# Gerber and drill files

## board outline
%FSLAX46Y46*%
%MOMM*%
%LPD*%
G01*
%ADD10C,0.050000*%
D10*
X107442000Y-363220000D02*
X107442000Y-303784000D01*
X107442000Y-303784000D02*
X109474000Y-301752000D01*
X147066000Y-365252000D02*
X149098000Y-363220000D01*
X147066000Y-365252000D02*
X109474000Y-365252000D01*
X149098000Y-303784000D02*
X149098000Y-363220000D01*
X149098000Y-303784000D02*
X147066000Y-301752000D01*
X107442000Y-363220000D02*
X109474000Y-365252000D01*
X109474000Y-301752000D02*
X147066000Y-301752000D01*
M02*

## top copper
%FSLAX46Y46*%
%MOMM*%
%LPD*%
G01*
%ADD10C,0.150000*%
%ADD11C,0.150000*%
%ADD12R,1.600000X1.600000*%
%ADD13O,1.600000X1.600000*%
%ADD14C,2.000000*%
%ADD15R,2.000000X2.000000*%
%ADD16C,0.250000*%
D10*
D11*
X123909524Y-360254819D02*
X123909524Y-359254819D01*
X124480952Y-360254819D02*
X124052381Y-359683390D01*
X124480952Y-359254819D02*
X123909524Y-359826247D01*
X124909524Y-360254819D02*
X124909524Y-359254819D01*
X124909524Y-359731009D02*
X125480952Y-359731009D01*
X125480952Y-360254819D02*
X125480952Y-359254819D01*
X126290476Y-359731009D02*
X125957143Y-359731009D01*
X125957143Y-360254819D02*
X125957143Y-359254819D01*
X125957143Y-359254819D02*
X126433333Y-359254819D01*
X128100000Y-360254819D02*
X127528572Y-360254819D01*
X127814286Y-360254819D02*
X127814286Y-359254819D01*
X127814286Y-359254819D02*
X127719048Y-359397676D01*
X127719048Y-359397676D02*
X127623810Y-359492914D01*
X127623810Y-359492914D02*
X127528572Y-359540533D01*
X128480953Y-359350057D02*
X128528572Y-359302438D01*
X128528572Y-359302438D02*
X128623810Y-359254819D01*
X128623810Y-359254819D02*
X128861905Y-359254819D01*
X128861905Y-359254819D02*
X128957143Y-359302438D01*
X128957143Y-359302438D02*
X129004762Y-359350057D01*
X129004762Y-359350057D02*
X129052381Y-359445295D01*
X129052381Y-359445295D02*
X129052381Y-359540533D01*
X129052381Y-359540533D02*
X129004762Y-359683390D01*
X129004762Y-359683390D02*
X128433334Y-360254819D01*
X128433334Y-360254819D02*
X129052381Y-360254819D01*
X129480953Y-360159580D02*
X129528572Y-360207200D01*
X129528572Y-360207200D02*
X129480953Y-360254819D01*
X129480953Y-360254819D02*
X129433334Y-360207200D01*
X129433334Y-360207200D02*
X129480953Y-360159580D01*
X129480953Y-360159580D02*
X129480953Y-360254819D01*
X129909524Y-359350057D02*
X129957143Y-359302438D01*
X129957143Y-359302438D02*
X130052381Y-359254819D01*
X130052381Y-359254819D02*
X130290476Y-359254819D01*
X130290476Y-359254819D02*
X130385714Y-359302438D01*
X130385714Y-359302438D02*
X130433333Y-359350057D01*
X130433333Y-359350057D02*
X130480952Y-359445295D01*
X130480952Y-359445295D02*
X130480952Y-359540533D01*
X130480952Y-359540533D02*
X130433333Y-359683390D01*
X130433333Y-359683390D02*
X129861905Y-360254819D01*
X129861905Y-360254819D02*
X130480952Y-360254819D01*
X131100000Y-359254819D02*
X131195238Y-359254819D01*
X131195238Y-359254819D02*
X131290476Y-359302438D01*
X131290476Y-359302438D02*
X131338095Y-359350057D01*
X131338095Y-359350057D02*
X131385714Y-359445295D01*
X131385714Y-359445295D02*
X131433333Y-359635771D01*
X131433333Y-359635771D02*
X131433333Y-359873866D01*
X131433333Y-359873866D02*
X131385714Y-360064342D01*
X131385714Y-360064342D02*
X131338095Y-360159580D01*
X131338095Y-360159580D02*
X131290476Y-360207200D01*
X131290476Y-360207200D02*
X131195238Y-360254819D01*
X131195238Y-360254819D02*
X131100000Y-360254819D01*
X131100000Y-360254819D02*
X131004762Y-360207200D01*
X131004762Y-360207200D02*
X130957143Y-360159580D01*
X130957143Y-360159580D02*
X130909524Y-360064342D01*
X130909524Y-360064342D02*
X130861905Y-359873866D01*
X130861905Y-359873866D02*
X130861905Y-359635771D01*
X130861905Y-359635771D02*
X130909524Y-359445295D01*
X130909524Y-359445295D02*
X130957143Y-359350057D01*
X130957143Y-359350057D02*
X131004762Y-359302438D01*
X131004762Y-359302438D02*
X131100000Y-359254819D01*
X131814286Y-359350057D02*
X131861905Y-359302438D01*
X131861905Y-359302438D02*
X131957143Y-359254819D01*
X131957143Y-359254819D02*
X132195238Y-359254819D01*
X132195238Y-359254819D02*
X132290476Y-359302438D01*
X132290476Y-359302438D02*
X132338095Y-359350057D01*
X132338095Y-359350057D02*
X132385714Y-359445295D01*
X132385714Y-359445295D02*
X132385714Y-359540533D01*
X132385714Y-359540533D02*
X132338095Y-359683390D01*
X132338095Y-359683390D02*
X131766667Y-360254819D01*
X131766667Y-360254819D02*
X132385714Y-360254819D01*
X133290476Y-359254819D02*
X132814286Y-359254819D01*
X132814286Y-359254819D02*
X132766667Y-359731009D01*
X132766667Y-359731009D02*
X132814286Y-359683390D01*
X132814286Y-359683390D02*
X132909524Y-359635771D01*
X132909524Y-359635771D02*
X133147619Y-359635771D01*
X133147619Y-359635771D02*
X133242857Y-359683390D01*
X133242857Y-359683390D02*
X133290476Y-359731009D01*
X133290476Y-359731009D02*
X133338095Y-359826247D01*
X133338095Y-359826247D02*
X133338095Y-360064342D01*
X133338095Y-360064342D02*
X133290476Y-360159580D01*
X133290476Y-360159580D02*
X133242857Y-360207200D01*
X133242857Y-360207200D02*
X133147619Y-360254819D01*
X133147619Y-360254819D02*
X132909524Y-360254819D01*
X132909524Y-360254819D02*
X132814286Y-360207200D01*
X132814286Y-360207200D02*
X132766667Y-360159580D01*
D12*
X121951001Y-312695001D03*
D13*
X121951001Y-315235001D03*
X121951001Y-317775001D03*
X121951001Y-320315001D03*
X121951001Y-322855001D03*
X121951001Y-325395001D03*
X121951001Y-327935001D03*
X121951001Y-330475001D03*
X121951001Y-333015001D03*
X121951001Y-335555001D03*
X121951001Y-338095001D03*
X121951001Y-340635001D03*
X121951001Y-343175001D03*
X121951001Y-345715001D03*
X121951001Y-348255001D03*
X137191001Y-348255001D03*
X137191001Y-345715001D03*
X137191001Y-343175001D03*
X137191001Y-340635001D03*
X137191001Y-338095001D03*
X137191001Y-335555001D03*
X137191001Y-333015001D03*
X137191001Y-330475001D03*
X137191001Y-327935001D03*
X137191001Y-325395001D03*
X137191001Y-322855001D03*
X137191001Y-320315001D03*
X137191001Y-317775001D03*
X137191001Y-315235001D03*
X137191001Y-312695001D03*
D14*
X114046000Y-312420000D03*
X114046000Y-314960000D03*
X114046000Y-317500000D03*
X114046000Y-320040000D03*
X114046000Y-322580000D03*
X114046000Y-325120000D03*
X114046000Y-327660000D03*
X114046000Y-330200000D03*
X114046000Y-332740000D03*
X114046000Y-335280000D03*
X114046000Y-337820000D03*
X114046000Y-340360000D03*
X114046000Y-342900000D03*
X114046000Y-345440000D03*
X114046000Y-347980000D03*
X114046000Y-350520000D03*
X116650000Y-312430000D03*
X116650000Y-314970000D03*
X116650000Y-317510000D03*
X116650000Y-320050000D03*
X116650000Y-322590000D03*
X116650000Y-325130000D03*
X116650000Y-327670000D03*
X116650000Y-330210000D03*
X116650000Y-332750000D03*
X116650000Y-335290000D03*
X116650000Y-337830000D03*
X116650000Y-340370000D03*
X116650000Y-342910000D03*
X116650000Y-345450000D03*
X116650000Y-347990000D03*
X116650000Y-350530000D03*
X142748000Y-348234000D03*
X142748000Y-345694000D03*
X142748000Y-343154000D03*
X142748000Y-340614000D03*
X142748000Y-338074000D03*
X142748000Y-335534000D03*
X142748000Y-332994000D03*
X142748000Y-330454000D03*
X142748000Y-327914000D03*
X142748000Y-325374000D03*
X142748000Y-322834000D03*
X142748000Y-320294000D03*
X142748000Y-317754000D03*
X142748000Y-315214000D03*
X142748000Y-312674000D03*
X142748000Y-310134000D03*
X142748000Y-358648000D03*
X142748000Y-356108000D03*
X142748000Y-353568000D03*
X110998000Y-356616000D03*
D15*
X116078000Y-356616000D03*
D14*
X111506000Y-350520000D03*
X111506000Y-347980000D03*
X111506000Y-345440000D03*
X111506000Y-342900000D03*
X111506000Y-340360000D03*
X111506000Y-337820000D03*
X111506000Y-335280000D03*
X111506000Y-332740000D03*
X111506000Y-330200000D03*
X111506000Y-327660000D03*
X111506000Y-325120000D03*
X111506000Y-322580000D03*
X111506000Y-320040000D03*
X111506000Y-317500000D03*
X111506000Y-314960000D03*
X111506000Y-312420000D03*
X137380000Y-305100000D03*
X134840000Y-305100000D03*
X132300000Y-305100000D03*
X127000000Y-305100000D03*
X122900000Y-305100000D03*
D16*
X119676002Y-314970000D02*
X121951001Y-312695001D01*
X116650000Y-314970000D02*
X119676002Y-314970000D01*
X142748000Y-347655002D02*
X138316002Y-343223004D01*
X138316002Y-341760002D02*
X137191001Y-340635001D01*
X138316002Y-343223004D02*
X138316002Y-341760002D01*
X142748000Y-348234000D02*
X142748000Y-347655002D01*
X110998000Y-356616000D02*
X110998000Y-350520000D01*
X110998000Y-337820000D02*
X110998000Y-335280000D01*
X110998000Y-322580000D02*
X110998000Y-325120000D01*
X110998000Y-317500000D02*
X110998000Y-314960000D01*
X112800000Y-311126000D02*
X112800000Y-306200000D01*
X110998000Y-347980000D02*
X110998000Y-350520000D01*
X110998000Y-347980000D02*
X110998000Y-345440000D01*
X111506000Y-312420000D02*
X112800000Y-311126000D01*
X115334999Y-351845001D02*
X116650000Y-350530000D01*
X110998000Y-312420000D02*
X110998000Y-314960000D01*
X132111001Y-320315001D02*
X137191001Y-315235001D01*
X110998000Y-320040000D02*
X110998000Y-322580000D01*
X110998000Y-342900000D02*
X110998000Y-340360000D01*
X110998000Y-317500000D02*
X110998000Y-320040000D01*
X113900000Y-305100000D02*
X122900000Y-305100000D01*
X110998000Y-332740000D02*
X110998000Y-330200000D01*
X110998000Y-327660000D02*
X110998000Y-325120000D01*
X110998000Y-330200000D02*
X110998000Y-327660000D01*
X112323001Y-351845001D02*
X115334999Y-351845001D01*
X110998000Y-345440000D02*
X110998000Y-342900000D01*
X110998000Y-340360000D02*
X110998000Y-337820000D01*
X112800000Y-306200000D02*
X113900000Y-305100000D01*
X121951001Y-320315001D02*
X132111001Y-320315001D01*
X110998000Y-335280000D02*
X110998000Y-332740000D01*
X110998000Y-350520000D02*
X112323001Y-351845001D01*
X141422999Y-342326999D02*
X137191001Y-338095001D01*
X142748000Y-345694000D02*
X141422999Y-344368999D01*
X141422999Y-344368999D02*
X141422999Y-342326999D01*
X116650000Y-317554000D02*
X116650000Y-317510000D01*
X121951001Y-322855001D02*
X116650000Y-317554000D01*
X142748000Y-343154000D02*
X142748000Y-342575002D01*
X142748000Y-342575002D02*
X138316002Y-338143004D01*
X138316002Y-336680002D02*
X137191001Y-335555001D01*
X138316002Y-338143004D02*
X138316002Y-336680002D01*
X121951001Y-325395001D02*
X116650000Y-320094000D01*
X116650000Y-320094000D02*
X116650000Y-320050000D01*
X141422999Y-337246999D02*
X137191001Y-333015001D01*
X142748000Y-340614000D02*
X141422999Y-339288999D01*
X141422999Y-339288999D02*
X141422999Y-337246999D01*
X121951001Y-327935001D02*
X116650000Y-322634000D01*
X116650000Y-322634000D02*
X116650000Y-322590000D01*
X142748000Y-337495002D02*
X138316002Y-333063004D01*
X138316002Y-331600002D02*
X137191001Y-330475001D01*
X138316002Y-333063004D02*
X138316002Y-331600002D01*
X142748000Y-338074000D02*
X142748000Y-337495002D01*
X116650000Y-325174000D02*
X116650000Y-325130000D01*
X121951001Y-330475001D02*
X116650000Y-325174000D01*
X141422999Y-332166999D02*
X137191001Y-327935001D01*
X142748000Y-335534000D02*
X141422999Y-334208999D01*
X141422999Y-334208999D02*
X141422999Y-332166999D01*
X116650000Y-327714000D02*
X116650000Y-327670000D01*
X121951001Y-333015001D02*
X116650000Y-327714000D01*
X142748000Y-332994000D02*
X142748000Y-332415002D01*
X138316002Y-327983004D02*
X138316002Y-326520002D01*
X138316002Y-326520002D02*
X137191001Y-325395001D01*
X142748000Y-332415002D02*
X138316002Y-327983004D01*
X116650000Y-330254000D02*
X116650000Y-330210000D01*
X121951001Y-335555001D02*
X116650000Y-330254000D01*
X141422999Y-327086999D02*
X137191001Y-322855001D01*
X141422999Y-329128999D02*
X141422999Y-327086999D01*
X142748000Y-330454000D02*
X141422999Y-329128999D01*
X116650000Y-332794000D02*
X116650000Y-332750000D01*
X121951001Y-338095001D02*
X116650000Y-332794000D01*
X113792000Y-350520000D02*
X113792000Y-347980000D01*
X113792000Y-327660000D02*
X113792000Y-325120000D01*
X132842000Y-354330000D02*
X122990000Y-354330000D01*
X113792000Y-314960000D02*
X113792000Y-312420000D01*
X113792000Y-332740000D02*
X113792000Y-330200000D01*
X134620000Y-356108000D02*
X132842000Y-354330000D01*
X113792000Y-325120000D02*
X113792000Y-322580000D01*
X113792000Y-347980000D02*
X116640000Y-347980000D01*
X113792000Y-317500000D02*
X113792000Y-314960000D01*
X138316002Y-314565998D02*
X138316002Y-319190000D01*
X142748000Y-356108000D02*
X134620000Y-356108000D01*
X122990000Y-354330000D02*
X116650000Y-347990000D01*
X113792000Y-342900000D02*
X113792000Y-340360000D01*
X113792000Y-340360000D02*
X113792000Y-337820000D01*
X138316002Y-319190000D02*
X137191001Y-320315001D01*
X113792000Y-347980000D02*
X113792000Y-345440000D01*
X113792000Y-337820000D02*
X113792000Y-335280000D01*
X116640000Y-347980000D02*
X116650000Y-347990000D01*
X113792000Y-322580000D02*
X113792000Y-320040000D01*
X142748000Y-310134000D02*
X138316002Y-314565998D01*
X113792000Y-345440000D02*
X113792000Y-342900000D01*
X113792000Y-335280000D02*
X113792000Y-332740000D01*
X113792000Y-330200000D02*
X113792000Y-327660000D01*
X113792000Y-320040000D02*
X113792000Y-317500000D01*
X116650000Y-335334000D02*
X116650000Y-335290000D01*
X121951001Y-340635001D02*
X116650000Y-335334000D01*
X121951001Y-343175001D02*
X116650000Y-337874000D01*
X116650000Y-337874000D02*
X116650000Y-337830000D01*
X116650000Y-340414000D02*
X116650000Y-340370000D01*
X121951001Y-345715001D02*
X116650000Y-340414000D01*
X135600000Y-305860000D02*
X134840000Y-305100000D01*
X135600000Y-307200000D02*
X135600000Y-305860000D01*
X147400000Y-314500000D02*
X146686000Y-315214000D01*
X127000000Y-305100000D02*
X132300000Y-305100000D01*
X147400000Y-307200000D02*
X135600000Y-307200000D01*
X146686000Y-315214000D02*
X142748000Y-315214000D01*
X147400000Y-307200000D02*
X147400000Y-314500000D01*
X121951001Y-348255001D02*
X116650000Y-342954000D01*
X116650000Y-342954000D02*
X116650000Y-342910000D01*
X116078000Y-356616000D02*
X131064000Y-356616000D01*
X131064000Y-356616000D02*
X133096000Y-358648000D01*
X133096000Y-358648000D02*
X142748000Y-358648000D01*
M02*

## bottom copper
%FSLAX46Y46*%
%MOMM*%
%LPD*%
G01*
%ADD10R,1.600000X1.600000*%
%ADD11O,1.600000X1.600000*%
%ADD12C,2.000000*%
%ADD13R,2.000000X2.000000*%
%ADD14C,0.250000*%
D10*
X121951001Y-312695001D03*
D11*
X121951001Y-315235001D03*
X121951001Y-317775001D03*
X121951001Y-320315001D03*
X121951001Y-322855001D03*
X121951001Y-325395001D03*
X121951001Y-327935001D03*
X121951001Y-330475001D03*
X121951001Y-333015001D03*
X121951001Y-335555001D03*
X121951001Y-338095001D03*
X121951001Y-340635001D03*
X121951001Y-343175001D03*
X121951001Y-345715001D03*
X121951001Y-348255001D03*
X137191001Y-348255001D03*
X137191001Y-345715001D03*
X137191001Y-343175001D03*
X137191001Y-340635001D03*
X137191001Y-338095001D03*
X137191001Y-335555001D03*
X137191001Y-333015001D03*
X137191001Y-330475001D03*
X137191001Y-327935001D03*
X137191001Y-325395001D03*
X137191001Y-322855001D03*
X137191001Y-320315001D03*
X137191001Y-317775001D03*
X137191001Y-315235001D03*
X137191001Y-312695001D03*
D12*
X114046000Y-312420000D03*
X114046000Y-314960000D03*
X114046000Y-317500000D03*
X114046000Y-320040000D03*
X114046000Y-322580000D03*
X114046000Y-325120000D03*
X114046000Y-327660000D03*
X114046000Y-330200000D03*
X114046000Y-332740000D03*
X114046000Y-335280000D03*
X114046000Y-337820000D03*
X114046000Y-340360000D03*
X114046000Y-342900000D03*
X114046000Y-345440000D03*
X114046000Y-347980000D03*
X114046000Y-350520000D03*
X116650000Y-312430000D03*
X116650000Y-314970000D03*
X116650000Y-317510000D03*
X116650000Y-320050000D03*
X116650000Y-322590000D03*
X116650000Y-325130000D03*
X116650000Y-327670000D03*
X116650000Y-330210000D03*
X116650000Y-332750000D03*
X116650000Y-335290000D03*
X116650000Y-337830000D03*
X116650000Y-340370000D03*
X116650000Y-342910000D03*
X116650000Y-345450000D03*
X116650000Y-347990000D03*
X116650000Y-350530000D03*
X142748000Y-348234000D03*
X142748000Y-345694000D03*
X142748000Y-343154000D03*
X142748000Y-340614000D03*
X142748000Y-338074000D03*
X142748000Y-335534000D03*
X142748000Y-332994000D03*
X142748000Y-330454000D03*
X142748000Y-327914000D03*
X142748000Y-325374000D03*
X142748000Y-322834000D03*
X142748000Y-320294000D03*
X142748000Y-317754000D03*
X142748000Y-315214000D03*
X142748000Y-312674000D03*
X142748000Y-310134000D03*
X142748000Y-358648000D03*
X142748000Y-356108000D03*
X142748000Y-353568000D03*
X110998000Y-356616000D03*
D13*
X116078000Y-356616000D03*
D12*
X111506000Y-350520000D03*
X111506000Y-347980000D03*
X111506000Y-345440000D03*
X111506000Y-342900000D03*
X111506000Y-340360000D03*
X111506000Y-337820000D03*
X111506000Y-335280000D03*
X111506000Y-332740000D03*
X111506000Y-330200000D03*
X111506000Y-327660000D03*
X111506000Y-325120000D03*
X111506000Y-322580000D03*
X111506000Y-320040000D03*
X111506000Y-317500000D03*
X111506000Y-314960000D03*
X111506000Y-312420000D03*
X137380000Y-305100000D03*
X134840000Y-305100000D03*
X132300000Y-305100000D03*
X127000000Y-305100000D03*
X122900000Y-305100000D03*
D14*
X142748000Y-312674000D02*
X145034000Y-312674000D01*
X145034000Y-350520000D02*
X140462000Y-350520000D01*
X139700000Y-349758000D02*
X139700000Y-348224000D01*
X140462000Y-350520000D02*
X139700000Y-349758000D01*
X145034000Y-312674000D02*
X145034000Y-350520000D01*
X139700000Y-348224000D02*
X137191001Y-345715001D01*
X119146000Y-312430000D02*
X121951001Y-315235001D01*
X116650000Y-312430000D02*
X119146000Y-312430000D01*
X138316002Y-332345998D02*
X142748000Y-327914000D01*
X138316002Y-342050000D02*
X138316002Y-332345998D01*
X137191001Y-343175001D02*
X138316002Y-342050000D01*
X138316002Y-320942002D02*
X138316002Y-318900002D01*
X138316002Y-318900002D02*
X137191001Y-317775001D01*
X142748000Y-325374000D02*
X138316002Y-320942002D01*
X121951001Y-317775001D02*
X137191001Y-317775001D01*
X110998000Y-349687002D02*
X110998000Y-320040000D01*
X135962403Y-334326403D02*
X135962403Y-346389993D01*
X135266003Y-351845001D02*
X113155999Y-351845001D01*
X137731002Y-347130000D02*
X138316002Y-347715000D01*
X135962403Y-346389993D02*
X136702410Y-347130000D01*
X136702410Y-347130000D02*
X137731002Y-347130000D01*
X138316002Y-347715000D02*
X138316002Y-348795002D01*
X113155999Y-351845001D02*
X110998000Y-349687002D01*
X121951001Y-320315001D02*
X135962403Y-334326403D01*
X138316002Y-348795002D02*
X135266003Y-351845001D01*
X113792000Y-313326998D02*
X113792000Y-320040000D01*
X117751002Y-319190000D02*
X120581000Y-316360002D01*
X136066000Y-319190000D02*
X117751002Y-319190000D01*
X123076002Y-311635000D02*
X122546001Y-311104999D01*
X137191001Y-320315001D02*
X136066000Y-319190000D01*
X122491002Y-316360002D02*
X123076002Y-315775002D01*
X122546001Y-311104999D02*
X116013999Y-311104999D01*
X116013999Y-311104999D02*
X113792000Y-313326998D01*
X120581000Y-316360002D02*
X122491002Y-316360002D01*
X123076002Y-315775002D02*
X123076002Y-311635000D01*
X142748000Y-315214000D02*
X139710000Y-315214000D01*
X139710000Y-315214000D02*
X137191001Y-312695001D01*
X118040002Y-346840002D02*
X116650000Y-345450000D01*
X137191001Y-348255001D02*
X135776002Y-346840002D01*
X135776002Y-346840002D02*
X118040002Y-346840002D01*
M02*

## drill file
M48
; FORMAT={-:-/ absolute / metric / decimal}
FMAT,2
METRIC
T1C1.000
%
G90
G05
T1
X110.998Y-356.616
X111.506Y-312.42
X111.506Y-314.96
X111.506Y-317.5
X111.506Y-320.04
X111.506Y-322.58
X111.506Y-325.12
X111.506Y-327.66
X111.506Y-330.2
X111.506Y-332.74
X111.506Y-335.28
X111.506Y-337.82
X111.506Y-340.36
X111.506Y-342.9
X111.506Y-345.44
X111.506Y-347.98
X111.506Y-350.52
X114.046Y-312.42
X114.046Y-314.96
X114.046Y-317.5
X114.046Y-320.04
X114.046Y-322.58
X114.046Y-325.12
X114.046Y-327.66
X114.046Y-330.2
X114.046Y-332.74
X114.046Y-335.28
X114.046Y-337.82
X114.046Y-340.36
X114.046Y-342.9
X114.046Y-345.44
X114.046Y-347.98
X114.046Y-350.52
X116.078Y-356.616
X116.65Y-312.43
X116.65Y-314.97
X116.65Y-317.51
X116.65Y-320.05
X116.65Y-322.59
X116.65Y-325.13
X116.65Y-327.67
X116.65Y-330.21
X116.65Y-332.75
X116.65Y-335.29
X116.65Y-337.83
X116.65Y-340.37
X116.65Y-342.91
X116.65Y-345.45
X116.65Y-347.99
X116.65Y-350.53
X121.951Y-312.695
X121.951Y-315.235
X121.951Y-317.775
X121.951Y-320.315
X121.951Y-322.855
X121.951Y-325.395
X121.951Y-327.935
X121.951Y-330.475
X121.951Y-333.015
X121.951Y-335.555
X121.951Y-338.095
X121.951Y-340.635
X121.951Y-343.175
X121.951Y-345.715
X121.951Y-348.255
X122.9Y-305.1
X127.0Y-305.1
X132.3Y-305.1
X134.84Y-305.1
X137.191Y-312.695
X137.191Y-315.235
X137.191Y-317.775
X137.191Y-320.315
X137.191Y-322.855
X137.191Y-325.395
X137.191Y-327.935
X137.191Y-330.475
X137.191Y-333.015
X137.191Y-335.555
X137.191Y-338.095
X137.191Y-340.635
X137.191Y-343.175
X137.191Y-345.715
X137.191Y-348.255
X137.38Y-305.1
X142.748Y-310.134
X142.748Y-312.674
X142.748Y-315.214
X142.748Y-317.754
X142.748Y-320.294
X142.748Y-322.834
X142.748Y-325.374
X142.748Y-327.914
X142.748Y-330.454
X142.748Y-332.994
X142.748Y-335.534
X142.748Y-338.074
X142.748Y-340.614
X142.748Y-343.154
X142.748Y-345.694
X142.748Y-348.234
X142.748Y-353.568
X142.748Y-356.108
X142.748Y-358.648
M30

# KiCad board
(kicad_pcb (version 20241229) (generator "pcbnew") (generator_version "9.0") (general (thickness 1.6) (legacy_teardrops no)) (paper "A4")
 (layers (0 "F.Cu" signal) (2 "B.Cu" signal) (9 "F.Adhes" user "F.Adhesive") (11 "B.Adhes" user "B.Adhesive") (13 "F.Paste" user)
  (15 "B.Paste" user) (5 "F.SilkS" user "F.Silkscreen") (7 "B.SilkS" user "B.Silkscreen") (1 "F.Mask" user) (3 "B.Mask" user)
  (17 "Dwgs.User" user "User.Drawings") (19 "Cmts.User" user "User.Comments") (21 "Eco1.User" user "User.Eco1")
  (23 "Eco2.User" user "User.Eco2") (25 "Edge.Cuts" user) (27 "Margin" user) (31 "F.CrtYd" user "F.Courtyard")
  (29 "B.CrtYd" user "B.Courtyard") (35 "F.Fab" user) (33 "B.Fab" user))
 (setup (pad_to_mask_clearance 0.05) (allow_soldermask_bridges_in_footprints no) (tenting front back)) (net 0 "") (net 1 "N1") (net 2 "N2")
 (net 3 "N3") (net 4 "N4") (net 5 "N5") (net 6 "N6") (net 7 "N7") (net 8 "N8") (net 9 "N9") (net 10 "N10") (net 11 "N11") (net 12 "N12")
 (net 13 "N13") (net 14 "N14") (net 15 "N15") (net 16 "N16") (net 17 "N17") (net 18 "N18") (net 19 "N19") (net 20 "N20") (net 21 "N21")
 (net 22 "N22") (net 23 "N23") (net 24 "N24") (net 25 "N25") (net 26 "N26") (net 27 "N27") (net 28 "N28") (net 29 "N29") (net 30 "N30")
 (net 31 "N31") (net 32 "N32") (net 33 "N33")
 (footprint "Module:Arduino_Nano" (layer "F.Cu") (at 121.951001 312.695001)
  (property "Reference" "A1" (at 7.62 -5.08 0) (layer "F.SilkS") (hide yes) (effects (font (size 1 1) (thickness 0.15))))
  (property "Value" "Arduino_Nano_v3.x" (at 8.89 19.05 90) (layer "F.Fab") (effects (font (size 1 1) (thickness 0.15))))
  (pad "1" thru_hole rect (at 0 0) (size 1.6 1.6) (drill 1) (layers "*.Cu" "*.Mask") (remove_unused_layers no) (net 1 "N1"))
  (pad "2" thru_hole oval (at 0 2.54) (size 1.6 1.6) (drill 1) (layers "*.Cu" "*.Mask") (remove_unused_layers no) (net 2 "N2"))
  (pad "3" thru_hole oval (at 0 5.08) (size 1.6 1.6) (drill 1) (layers "*.Cu" "*.Mask") (remove_unused_layers no) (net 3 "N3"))
  (pad "4" thru_hole oval (at 0 7.62) (size 1.6 1.6) (drill 1) (layers "*.Cu" "*.Mask") (remove_unused_layers no) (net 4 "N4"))
  (pad "5" thru_hole oval (at 0 10.16) (size 1.6 1.6) (drill 1) (layers "*.Cu" "*.Mask") (remove_unused_layers no) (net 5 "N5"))
  (pad "6" thru_hole oval (at 0 12.7) (size 1.6 1.6) (drill 1) (layers "*.Cu" "*.Mask") (remove_unused_layers no) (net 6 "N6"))
  (pad "7" thru_hole oval (at 0 15.24) (size 1.6 1.6) (drill 1) (layers "*.Cu" "*.Mask") (remove_unused_layers no) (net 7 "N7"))
  (pad "8" thru_hole oval (at 0 17.78) (size 1.6 1.6) (drill 1) (layers "*.Cu" "*.Mask") (remove_unused_layers no) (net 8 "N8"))
  (pad "9" thru_hole oval (at 0 20.32) (size 1.6 1.6) (drill 1) (layers "*.Cu" "*.Mask") (remove_unused_layers no) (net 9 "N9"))
  (pad "10" thru_hole oval (at 0 22.86) (size 1.6 1.6) (drill 1) (layers "*.Cu" "*.Mask") (remove_unused_layers no) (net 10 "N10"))
  (pad "11" thru_hole oval (at 0 25.4) (size 1.6 1.6) (drill 1) (layers "*.Cu" "*.Mask") (remove_unused_layers no) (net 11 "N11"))
  (pad "12" thru_hole oval (at 0 27.94) (size 1.6 1.6) (drill 1) (layers "*.Cu" "*.Mask") (remove_unused_layers no) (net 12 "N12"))
  (pad "13" thru_hole oval (at 0 30.48) (size 1.6 1.6) (drill 1) (layers "*.Cu" "*.Mask") (remove_unused_layers no) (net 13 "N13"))
  (pad "14" thru_hole oval (at 0 33.02) (size 1.6 1.6) (drill 1) (layers "*.Cu" "*.Mask") (remove_unused_layers no) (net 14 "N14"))
  (pad "15" thru_hole oval (at 0 35.56) (size 1.6 1.6) (drill 1) (layers "*.Cu" "*.Mask") (remove_unused_layers no) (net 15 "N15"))
  (pad "16" thru_hole oval (at 15.24 35.56) (size 1.6 1.6) (drill 1) (layers "*.Cu" "*.Mask") (remove_unused_layers no) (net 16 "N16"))
  (pad "17" thru_hole oval (at 15.24 33.02) (size 1.6 1.6) (drill 1) (layers "*.Cu" "*.Mask") (remove_unused_layers no) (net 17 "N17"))
  (pad "18" thru_hole oval (at 15.24 30.48) (size 1.6 1.6) (drill 1) (layers "*.Cu" "*.Mask") (remove_unused_layers no) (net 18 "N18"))
  (pad "19" thru_hole oval (at 15.24 27.94) (size 1.6 1.6) (drill 1) (layers "*.Cu" "*.Mask") (remove_unused_layers no) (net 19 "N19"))
  (pad "20" thru_hole oval (at 15.24 25.4) (size 1.6 1.6) (drill 1) (layers "*.Cu" "*.Mask") (remove_unused_layers no) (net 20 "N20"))
  (pad "21" thru_hole oval (at 15.24 22.86) (size 1.6 1.6) (drill 1) (layers "*.Cu" "*.Mask") (remove_unused_layers no) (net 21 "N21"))
  (pad "22" thru_hole oval (at 15.24 20.32) (size 1.6 1.6) (drill 1) (layers "*.Cu" "*.Mask") (remove_unused_layers no) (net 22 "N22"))
  (pad "23" thru_hole oval (at 15.24 17.78) (size 1.6 1.6) (drill 1) (layers "*.Cu" "*.Mask") (remove_unused_layers no) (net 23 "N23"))
  (pad "24" thru_hole oval (at 15.24 15.24) (size 1.6 1.6) (drill 1) (layers "*.Cu" "*.Mask") (remove_unused_layers no) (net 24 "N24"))
  (pad "25" thru_hole oval (at 15.24 12.7) (size 1.6 1.6) (drill 1) (layers "*.Cu" "*.Mask") (remove_unused_layers no) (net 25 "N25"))
  (pad "26" thru_hole oval (at 15.24 10.16) (size 1.6 1.6) (drill 1) (layers "*.Cu" "*.Mask") (remove_unused_layers no) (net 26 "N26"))
  (pad "27" thru_hole oval (at 15.24 7.62) (size 1.6 1.6) (drill 1) (layers "*.Cu" "*.Mask") (remove_unused_layers no) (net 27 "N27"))
  (pad "28" thru_hole oval (at 15.24 5.08) (size 1.6 1.6) (drill 1) (layers "*.Cu" "*.Mask") (remove_unused_layers no) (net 3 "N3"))
  (pad "29" thru_hole oval (at 15.24 2.54) (size 1.6 1.6) (drill 1) (layers "*.Cu" "*.Mask") (remove_unused_layers no) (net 4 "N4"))
  (pad "30" thru_hole oval (at 15.24 0) (size 1.6 1.6) (drill 1) (layers "*.Cu" "*.Mask") (remove_unused_layers no) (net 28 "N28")))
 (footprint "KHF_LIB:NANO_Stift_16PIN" (layer "F.Cu") (at 114.046 312.42 -90)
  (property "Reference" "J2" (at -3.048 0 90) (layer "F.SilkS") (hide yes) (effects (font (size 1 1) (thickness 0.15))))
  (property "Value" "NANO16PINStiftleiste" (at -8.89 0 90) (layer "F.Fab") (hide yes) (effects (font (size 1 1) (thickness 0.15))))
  (pad "1" thru_hole circle (at 0 0 270) (size 2 2) (drill 1) (layers "*.Cu" "*.Mask") (remove_unused_layers no) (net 27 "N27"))
  (pad "2" thru_hole circle (at 2.54 0 270) (size 2 2) (drill 1) (layers "*.Cu" "*.Mask") (remove_unused_layers no) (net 27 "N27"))
  (pad "3" thru_hole circle (at 5.08 0 270) (size 2 2) (drill 1) (layers "*.Cu" "*.Mask") (remove_unused_layers no) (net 27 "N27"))
  (pad "4" thru_hole circle (at 7.62 0 270) (size 2 2) (drill 1) (layers "*.Cu" "*.Mask") (remove_unused_layers no) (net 27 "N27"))
  (pad "5" thru_hole circle (at 10.16 0 270) (size 2 2) (drill 1) (layers "*.Cu" "*.Mask") (remove_unused_layers no) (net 27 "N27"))
  (pad "6" thru_hole circle (at 12.7 0 270) (size 2 2) (drill 1) (layers "*.Cu" "*.Mask") (remove_unused_layers no) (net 27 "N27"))
  (pad "7" thru_hole circle (at 15.24 0 270) (size 2 2) (drill 1) (layers "*.Cu" "*.Mask") (remove_unused_layers no) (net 27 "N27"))
  (pad "8" thru_hole circle (at 17.78 0 270) (size 2 2) (drill 1) (layers "*.Cu" "*.Mask") (remove_unused_layers no) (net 27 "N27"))
  (pad "9" thru_hole circle (at 20.32 0 270) (size 2 2) (drill 1) (layers "*.Cu" "*.Mask") (remove_unused_layers no) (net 27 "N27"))
  (pad "10" thru_hole circle (at 22.86 0 270) (size 2 2) (drill 1) (layers "*.Cu" "*.Mask") (remove_unused_layers no) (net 27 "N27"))
  (pad "11" thru_hole circle (at 25.4 0 270) (size 2 2) (drill 1) (layers "*.Cu" "*.Mask") (remove_unused_layers no) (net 27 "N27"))
  (pad "12" thru_hole circle (at 27.94 0 270) (size 2 2) (drill 1) (layers "*.Cu" "*.Mask") (remove_unused_layers no) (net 27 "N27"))
  (pad "13" thru_hole circle (at 30.48 0 270) (size 2 2) (drill 1) (layers "*.Cu" "*.Mask") (remove_unused_layers no) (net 27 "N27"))
  (pad "14" thru_hole circle (at 33.02 0 270) (size 2 2) (drill 1) (layers "*.Cu" "*.Mask") (remove_unused_layers no) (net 27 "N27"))
  (pad "15" thru_hole circle (at 35.56 0 270) (size 2 2) (drill 1) (layers "*.Cu" "*.Mask") (remove_unused_layers no) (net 27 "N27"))
  (pad "16" thru_hole circle (at 38.1 0 270) (size 2 2) (drill 1) (layers "*.Cu" "*.Mask") (remove_unused_layers no) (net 27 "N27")))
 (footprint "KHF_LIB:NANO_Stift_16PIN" (layer "F.Cu") (at 116.65 312.43 -90)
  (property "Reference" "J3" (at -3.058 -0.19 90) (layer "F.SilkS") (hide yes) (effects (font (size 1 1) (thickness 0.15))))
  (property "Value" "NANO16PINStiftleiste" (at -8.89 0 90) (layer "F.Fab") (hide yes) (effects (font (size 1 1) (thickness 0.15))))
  (pad "1" thru_hole circle (at 0 0 270) (size 2 2) (drill 1) (layers "*.Cu" "*.Mask") (remove_unused_layers no) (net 2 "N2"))
  (pad "2" thru_hole circle (at 2.54 0 270) (size 2 2) (drill 1) (layers "*.Cu" "*.Mask") (remove_unused_layers no) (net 1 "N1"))
  (pad "3" thru_hole circle (at 5.08 0 270) (size 2 2) (drill 1) (layers "*.Cu" "*.Mask") (remove_unused_layers no) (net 5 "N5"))
  (pad "4" thru_hole circle (at 7.62 0 270) (size 2 2) (drill 1) (layers "*.Cu" "*.Mask") (remove_unused_layers no) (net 6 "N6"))
  (pad "5" thru_hole circle (at 10.16 0 270) (size 2 2) (drill 1) (layers "*.Cu" "*.Mask") (remove_unused_layers no) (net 7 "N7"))
  (pad "6" thru_hole circle (at 12.7 0 270) (size 2 2) (drill 1) (layers "*.Cu" "*.Mask") (remove_unused_layers no) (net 8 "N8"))
  (pad "7" thru_hole circle (at 15.24 0 270) (size 2 2) (drill 1) (layers "*.Cu" "*.Mask") (remove_unused_layers no) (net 9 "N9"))
  (pad "8" thru_hole circle (at 17.78 0 270) (size 2 2) (drill 1) (layers "*.Cu" "*.Mask") (remove_unused_layers no) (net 10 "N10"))
  (pad "9" thru_hole circle (at 20.32 0 270) (size 2 2) (drill 1) (layers "*.Cu" "*.Mask") (remove_unused_layers no) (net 11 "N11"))
  (pad "10" thru_hole circle (at 22.86 0 270) (size 2 2) (drill 1) (layers "*.Cu" "*.Mask") (remove_unused_layers no) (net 12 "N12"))
  (pad "11" thru_hole circle (at 25.4 0 270) (size 2 2) (drill 1) (layers "*.Cu" "*.Mask") (remove_unused_layers no) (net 13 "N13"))
  (pad "12" thru_hole circle (at 27.94 0 270) (size 2 2) (drill 1) (layers "*.Cu" "*.Mask") (remove_unused_layers no) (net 14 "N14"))
  (pad "13" thru_hole circle (at 30.48 0 270) (size 2 2) (drill 1) (layers "*.Cu" "*.Mask") (remove_unused_layers no) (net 15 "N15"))
  (pad "14" thru_hole circle (at 33.02 0 270) (size 2 2) (drill 1) (layers "*.Cu" "*.Mask") (remove_unused_layers no) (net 16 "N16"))
  (pad "15" thru_hole circle (at 35.56 0 270) (size 2 2) (drill 1) (layers "*.Cu" "*.Mask") (remove_unused_layers no) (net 27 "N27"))
  (pad "16" thru_hole circle (at 38.1 0 270) (size 2 2) (drill 1) (layers "*.Cu" "*.Mask") (remove_unused_layers no) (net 4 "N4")))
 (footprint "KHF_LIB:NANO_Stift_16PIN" (layer "F.Cu") (at 142.748 348.234 90)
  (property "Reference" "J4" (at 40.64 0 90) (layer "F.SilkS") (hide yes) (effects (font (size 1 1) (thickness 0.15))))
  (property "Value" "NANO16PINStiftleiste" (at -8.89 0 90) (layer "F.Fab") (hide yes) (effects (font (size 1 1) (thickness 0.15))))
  (pad "1" thru_hole circle (at 0 0 90) (size 2 2) (drill 1) (layers "*.Cu" "*.Mask") (remove_unused_layers no) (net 19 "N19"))
  (pad "2" thru_hole circle (at 2.54 0 90) (size 2 2) (drill 1) (layers "*.Cu" "*.Mask") (remove_unused_layers no) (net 20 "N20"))
  (pad "3" thru_hole circle (at 5.08 0 90) (size 2 2) (drill 1) (layers "*.Cu" "*.Mask") (remove_unused_layers no) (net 21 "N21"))
  (pad "4" thru_hole circle (at 7.62 0 90) (size 2 2) (drill 1) (layers "*.Cu" "*.Mask") (remove_unused_layers no) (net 22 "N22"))
  (pad "5" thru_hole circle (at 10.16 0 90) (size 2 2) (drill 1) (layers "*.Cu" "*.Mask") (remove_unused_layers no) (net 23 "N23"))
  (pad "6" thru_hole circle (at 12.7 0 90) (size 2 2) (drill 1) (layers "*.Cu" "*.Mask") (remove_unused_layers no) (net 24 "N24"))
  (pad "7" thru_hole circle (at 15.24 0 90) (size 2 2) (drill 1) (layers "*.Cu" "*.Mask") (remove_unused_layers no) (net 25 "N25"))
  (pad "8" thru_hole circle (at 17.78 0 90) (size 2 2) (drill 1) (layers "*.Cu" "*.Mask") (remove_unused_layers no) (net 26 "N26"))
  (pad "9" thru_hole circle (at 20.32 0 90) (size 2 2) (drill 1) (layers "*.Cu" "*.Mask") (remove_unused_layers no) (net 18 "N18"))
  (pad "10" thru_hole circle (at 22.86 0 90) (size 2 2) (drill 1) (layers "*.Cu" "*.Mask") (remove_unused_layers no) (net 3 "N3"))
  (pad "11" thru_hole circle (at 25.4 0 90) (size 2 2) (drill 1) (layers "*.Cu" "*.Mask") (remove_unused_layers no) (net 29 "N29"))
  (pad "12" thru_hole circle (at 27.94 0 90) (size 2 2) (drill 1) (layers "*.Cu" "*.Mask") (remove_unused_layers no) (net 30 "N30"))
  (pad "13" thru_hole circle (at 30.48 0 90) (size 2 2) (drill 1) (layers "*.Cu" "*.Mask") (remove_unused_layers no) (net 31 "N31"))
  (pad "14" thru_hole circle (at 33.02 0 90) (size 2 2) (drill 1) (layers "*.Cu" "*.Mask") (remove_unused_layers no) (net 28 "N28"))
  (pad "15" thru_hole circle (at 35.56 0 90) (size 2 2) (drill 1) (layers "*.Cu" "*.Mask") (remove_unused_layers no) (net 17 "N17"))
  (pad "16" thru_hole circle (at 38.1 0 90) (size 2 2) (drill 1) (layers "*.Cu" "*.Mask") (remove_unused_layers no) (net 27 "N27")))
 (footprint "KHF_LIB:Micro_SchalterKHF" (layer "F.Cu") (at 142.748 358.648 90)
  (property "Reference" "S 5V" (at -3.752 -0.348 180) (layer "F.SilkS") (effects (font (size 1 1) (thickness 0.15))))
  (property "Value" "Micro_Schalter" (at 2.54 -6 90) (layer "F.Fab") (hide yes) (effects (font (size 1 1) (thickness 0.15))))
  (pad "1" thru_hole circle (at 0 0 90) (size 2 2) (drill 1) (layers "*.Cu" "*.Mask") (remove_unused_layers no) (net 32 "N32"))
  (pad "2" thru_hole circle (at 2.54 0 90) (size 2 2) (drill 1) (layers "*.Cu" "*.Mask") (remove_unused_layers no) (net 27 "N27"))
  (pad "3" thru_hole circle (at 5.08 0 90) (size 2 2) (drill 1) (layers "*.Cu" "*.Mask") (remove_unused_layers no) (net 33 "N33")))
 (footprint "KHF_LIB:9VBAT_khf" (layer "F.Cu") (at 110.998 356.616)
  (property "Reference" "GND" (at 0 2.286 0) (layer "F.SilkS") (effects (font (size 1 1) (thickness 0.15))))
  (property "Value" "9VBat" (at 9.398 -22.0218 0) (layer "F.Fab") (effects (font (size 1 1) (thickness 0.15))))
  (pad "1" thru_hole circle (at 0 0) (size 2 2) (drill 1) (layers "*.Cu" "*.Mask") (remove_unused_layers no) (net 4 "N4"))
  (pad "2" thru_hole rect (at 5.08 0) (size 2 2) (drill 1) (layers "*.Cu" "*.Mask") (remove_unused_layers no) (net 32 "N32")))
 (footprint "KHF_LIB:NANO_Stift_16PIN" (layer "F.Cu") (at 111.506 350.52 90)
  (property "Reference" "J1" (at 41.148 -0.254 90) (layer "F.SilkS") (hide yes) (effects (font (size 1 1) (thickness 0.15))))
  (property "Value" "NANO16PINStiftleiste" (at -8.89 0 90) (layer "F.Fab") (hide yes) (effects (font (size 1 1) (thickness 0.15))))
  (pad "1" thru_hole circle (at 0 0 90) (size 2 2) (drill 1) (layers "*.Cu" "*.Mask") (remove_unused_layers no) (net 4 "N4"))
  (pad "2" thru_hole circle (at 2.54 0 90) (size 2 2) (drill 1) (layers "*.Cu" "*.Mask") (remove_unused_layers no) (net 4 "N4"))
  (pad "3" thru_hole circle (at 5.08 0 90) (size 2 2) (drill 1) (layers "*.Cu" "*.Mask") (remove_unused_layers no) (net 4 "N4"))
  (pad "4" thru_hole circle (at 7.62 0 90) (size 2 2) (drill 1) (layers "*.Cu" "*.Mask") (remove_unused_layers no) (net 4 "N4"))
  (pad "5" thru_hole circle (at 10.16 0 90) (size 2 2) (drill 1) (layers "*.Cu" "*.Mask") (remove_unused_layers no) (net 4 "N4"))
  (pad "6" thru_hole circle (at 12.7 0 90) (size 2 2) (drill 1) (layers "*.Cu" "*.Mask") (remove_unused_layers no) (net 4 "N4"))
  (pad "7" thru_hole circle (at 15.24 0 90) (size 2 2) (drill 1) (layers "*.Cu" "*.Mask") (remove_unused_layers no) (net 4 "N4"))
  (pad "8" thru_hole circle (at 17.78 0 90) (size 2 2) (drill 1) (layers "*.Cu" "*.Mask") (remove_unused_layers no) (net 4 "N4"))
  (pad "9" thru_hole circle (at 20.32 0 90) (size 2 2) (drill 1) (layers "*.Cu" "*.Mask") (remove_unused_layers no) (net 4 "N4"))
  (pad "10" thru_hole circle (at 22.86 0 90) (size 2 2) (drill 1) (layers "*.Cu" "*.Mask") (remove_unused_layers no) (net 4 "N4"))
  (pad "11" thru_hole circle (at 25.4 0 90) (size 2 2) (drill 1) (layers "*.Cu" "*.Mask") (remove_unused_layers no) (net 4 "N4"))
  (pad "12" thru_hole circle (at 27.94 0 90) (size 2 2) (drill 1) (layers "*.Cu" "*.Mask") (remove_unused_layers no) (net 4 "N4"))
  (pad "13" thru_hole circle (at 30.48 0 90) (size 2 2) (drill 1) (layers "*.Cu" "*.Mask") (remove_unused_layers no) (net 4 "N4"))
  (pad "14" thru_hole circle (at 33.02 0 90) (size 2 2) (drill 1) (layers "*.Cu" "*.Mask") (remove_unused_layers no) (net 4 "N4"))
  (pad "15" thru_hole circle (at 35.56 0 90) (size 2 2) (drill 1) (layers "*.Cu" "*.Mask") (remove_unused_layers no) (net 4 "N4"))
  (pad "16" thru_hole circle (at 38.1 0 90) (size 2 2) (drill 1) (layers "*.Cu" "*.Mask") (remove_unused_layers no) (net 4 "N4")))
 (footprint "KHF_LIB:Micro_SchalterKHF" (layer "F.Cu") (at 137.38 305.1 180)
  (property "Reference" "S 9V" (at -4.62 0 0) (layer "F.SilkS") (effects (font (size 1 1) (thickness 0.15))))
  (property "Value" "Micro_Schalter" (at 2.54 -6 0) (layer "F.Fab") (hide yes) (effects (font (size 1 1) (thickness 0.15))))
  (pad "1" thru_hole circle (at 0 0 180) (size 2 2) (drill 1) (layers "*.Cu" "*.Mask") (remove_unused_layers no))
  (pad "2" thru_hole circle (at 2.54 0 180) (size 2 2) (drill 1) (layers "*.Cu" "*.Mask") (remove_unused_layers no) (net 28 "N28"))
  (pad "3" thru_hole circle (at 5.08 0 180) (size 2 2) (drill 1) (layers "*.Cu" "*.Mask") (remove_unused_layers no) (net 28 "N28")))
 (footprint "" (layer "F.Cu") (at 127 305.1)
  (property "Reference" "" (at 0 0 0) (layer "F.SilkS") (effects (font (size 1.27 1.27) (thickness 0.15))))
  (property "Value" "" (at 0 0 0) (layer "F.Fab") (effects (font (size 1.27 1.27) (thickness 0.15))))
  (pad "16" thru_hole circle (at 0 0 90) (size 2 2) (drill 1) (layers "*.Cu" "*.Mask") (remove_unused_layers no) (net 28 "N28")))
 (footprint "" (layer "F.Cu") (at 122.9 305.1)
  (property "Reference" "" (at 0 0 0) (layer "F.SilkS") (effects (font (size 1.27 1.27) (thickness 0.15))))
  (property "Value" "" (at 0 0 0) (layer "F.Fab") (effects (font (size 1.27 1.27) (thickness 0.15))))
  (pad "16" thru_hole circle (at 0 0 90) (size 2 2) (drill 1) (layers "*.Cu" "*.Mask") (remove_unused_layers no) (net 4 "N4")))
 (gr_line (start 107.442 363.22) (end 107.442 303.784) (stroke (width 0.05) (type solid)) (layer "Edge.Cuts"))
 (gr_line (start 107.442 303.784) (end 109.474 301.752) (stroke (width 0.05) (type solid)) (layer "Edge.Cuts"))
 (gr_line (start 147.066 365.252) (end 149.098 363.22) (stroke (width 0.05) (type solid)) (layer "Edge.Cuts"))
 (gr_line (start 147.066 365.252) (end 109.474 365.252) (stroke (width 0.05) (type solid)) (layer "Edge.Cuts"))
 (gr_line (start 149.098 303.784) (end 149.098 363.22) (stroke (width 0.05) (type solid)) (layer "Edge.Cuts"))
 (gr_line (start 149.098 303.784) (end 147.066 301.752) (stroke (width 0.05) (type solid)) (layer "Edge.Cuts"))
 (gr_line (start 107.442 363.22) (end 109.474 365.252) (stroke (width 0.05) (type solid)) (layer "Edge.Cuts"))
 (gr_line (start 109.474 301.752) (end 147.066 301.752) (stroke (width 0.05) (type solid)) (layer "Edge.Cuts"))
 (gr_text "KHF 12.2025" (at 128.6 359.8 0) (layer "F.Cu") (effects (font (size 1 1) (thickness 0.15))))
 (segment (start 119.676002 314.97) (end 121.951001 312.695001) (width 0.25) (layer "F.Cu") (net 1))
 (segment (start 116.65 314.97) (end 119.676002 314.97) (width 0.25) (layer "F.Cu") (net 1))
 (segment (start 142.748 312.674) (end 145.034 312.674) (width 0.25) (layer "B.Cu") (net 17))
 (segment (start 145.034 350.52) (end 140.462 350.52) (width 0.25) (layer "B.Cu") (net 17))
 (segment (start 139.7 349.758) (end 139.7 348.224) (width 0.25) (layer "B.Cu") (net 17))
 (segment (start 140.462 350.52) (end 139.7 349.758) (width 0.25) (layer "B.Cu") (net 17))
 (segment (start 145.034 312.674) (end 145.034 350.52) (width 0.25) (layer "B.Cu") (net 17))
 (segment (start 139.7 348.224) (end 137.191001 345.715001) (width 0.25) (layer "B.Cu") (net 17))
 (segment (start 119.146 312.43) (end 121.951001 315.235001) (width 0.25) (layer "B.Cu") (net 2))
 (segment (start 116.65 312.43) (end 119.146 312.43) (width 0.25) (layer "B.Cu") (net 2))
 (segment (start 138.316002 332.345998) (end 142.748 327.914) (width 0.25) (layer "B.Cu") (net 18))
 (segment (start 138.316002 342.05) (end 138.316002 332.345998) (width 0.25) (layer "B.Cu") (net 18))
 (segment (start 137.191001 343.175001) (end 138.316002 342.05) (width 0.25) (layer "B.Cu") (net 18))
 (segment (start 138.316002 320.942002) (end 138.316002 318.900002) (width 0.25) (layer "B.Cu") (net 3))
 (segment (start 138.316002 318.900002) (end 137.191001 317.775001) (width 0.25) (layer "B.Cu") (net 3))
 (segment (start 142.748 325.374) (end 138.316002 320.942002) (width 0.25) (layer "B.Cu") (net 3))
 (segment (start 121.951001 317.775001) (end 137.191001 317.775001) (width 0.25) (layer "B.Cu") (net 3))
 (segment (start 142.748 347.655002) (end 138.316002 343.223004) (width 0.25) (layer "F.Cu") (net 19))
 (segment (start 138.316002 341.760002) (end 137.191001 340.635001) (width 0.25) (layer "F.Cu") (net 19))
 (segment (start 138.316002 343.223004) (end 138.316002 341.760002) (width 0.25) (layer "F.Cu") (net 19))
 (segment (start 142.748 348.234) (end 142.748 347.655002) (width 0.25) (layer "F.Cu") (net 19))
 (segment (start 110.998 356.616) (end 110.998 350.52) (width 0.25) (layer "F.Cu") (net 4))
 (segment (start 110.998 337.82) (end 110.998 335.28) (width 0.25) (layer "F.Cu") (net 4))
 (segment (start 110.998 322.58) (end 110.998 325.12) (width 0.25) (layer "F.Cu") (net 4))
 (segment (start 110.998 317.5) (end 110.998 314.96) (width 0.25) (layer "F.Cu") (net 4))
 (segment (start 112.8 311.126) (end 112.8 306.2) (width 0.25) (layer "F.Cu") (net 4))
 (segment (start 110.998 347.98) (end 110.998 350.52) (width 0.25) (layer "F.Cu") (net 4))
 (segment (start 110.998 347.98) (end 110.998 345.44) (width 0.25) (layer "F.Cu") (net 4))
 (segment (start 111.506 312.42) (end 112.8 311.126) (width 0.25) (layer "F.Cu") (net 4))
 (segment (start 115.334999 351.845001) (end 116.65 350.53) (width 0.25) (layer "F.Cu") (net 4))
 (segment (start 110.998 312.42) (end 110.998 314.96) (width 0.25) (layer "F.Cu") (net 4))
 (segment (start 132.111001 320.315001) (end 137.191001 315.235001) (width 0.25) (layer "F.Cu") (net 4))
 (segment (start 110.998 320.04) (end 110.998 322.58) (width 0.25) (layer "F.Cu") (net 4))
 (segment (start 110.998 342.9) (end 110.998 340.36) (width 0.25) (layer "F.Cu") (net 4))
 (segment (start 110.998 317.5) (end 110.998 320.04) (width 0.25) (layer "F.Cu") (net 4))
 (segment (start 113.9 305.1) (end 122.9 305.1) (width 0.25) (layer "F.Cu") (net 4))
 (segment (start 110.998 332.74) (end 110.998 330.2) (width 0.25) (layer "F.Cu") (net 4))
 (segment (start 110.998 327.66) (end 110.998 325.12) (width 0.25) (layer "F.Cu") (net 4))
 (segment (start 110.998 330.2) (end 110.998 327.66) (width 0.25) (layer "F.Cu") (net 4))
 (segment (start 112.323001 351.845001) (end 115.334999 351.845001) (width 0.25) (layer "F.Cu") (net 4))
 (segment (start 110.998 345.44) (end 110.998 342.9) (width 0.25) (layer "F.Cu") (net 4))
 (segment (start 110.998 340.36) (end 110.998 337.82) (width 0.25) (layer "F.Cu") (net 4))
 (segment (start 112.8 306.2) (end 113.9 305.1) (width 0.25) (layer "F.Cu") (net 4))
 (segment (start 121.951001 320.315001) (end 132.111001 320.315001) (width 0.25) (layer "F.Cu") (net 4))
 (segment (start 110.998 335.28) (end 110.998 332.74) (width 0.25) (layer "F.Cu") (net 4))
 (segment (start 110.998 350.52) (end 112.323001 351.845001) (width 0.25) (layer "F.Cu") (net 4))
 (segment (start 110.998 349.687002) (end 110.998 320.04) (width 0.25) (layer "B.Cu") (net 4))
 (segment (start 135.962403 334.326403) (end 135.962403 346.389993) (width 0.25) (layer "B.Cu") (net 4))
 (segment (start 135.266003 351.845001) (end 113.155999 351.845001) (width 0.25) (layer "B.Cu") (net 4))
 (segment (start 137.731002 347.13) (end 138.316002 347.715) (width 0.25) (layer "B.Cu") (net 4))
 (segment (start 135.962403 346.389993) (end 136.70241 347.13) (width 0.25) (layer "B.Cu") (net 4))
 (segment (start 136.70241 347.13) (end 137.731002 347.13) (width 0.25) (layer "B.Cu") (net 4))
 (segment (start 138.316002 347.715) (end 138.316002 348.795002) (width 0.25) (layer "B.Cu") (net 4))
 (segment (start 113.155999 351.845001) (end 110.998 349.687002) (width 0.25) (layer "B.Cu") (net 4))
 (segment (start 121.951001 320.315001) (end 135.962403 334.326403) (width 0.25) (layer "B.Cu") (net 4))
 (segment (start 138.316002 348.795002) (end 135.266003 351.845001) (width 0.25) (layer "B.Cu") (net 4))
 (segment (start 141.422999 342.326999) (end 137.191001 338.095001) (width 0.25) (layer "F.Cu") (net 20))
 (segment (start 142.748 345.694) (end 141.422999 344.368999) (width 0.25) (layer "F.Cu") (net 20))
 (segment (start 141.422999 344.368999) (end 141.422999 342.326999) (width 0.25) (layer "F.Cu") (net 20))
 (segment (start 116.65 317.554) (end 116.65 317.51) (width 0.25) (layer "F.Cu") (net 5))
 (segment (start 121.951001 322.855001) (end 116.65 317.554) (width 0.25) (layer "F.Cu") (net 5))
 (segment (start 142.748 343.154) (end 142.748 342.575002) (width 0.25) (layer "F.Cu") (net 21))
 (segment (start 142.748 342.575002) (end 138.316002 338.143004) (width 0.25) (layer "F.Cu") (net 21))
 (segment (start 138.316002 336.680002) (end 137.191001 335.555001) (width 0.25) (layer "F.Cu") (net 21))
 (segment (start 138.316002 338.143004) (end 138.316002 336.680002) (width 0.25) (layer "F.Cu") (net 21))
 (segment (start 121.951001 325.395001) (end 116.65 320.094) (width 0.25) (layer "F.Cu") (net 6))
 (segment (start 116.65 320.094) (end 116.65 320.05) (width 0.25) (layer "F.Cu") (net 6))
 (segment (start 141.422999 337.246999) (end 137.191001 333.015001) (width 0.25) (layer "F.Cu") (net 22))
 (segment (start 142.748 340.614) (end 141.422999 339.288999) (width 0.25) (layer "F.Cu") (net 22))
 (segment (start 141.422999 339.288999) (end 141.422999 337.246999) (width 0.25) (layer "F.Cu") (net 22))
 (segment (start 121.951001 327.935001) (end 116.65 322.634) (width 0.25) (layer "F.Cu") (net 7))
 (segment (start 116.65 322.634) (end 116.65 322.59) (width 0.25) (layer "F.Cu") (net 7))
 (segment (start 142.748 337.495002) (end 138.316002 333.063004) (width 0.25) (layer "F.Cu") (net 23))
 (segment (start 138.316002 331.600002) (end 137.191001 330.475001) (width 0.25) (layer "F.Cu") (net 23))
 (segment (start 138.316002 333.063004) (end 138.316002 331.600002) (width 0.25) (layer "F.Cu") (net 23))
 (segment (start 142.748 338.074) (end 142.748 337.495002) (width 0.25) (layer "F.Cu") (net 23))
 (segment (start 116.65 325.174) (end 116.65 325.13) (width 0.25) (layer "F.Cu") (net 8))
 (segment (start 121.951001 330.475001) (end 116.65 325.174) (width 0.25) (layer "F.Cu") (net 8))
 (segment (start 141.422999 332.166999) (end 137.191001 327.935001) (width 0.25) (layer "F.Cu") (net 24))
 (segment (start 142.748 335.534) (end 141.422999 334.208999) (width 0.25) (layer "F.Cu") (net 24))
 (segment (start 141.422999 334.208999) (end 141.422999 332.166999) (width 0.25) (layer "F.Cu") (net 24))
 (segment (start 116.65 327.714) (end 116.65 327.67) (width 0.25) (layer "F.Cu") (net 9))
 (segment (start 121.951001 333.015001) (end 116.65 327.714) (width 0.25) (layer "F.Cu") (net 9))
 (segment (start 142.748 332.994) (end 142.748 332.415002) (width 0.25) (layer "F.Cu") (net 25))
 (segment (start 138.316002 327.983004) (end 138.316002 326.520002) (width 0.25) (layer "F.Cu") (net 25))
 (segment (start 138.316002 326.520002) (end 137.191001 325.395001) (width 0.25) (layer "F.Cu") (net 25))
 (segment (start 142.748 332.415002) (end 138.316002 327.983004) (width 0.25) (layer "F.Cu") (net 25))
 (segment (start 116.65 330.254) (end 116.65 330.21) (width 0.25) (layer "F.Cu") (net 10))
 (segment (start 121.951001 335.555001) (end 116.65 330.254) (width 0.25) (layer "F.Cu") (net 10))
 (segment (start 141.422999 327.086999) (end 137.191001 322.855001) (width 0.25) (layer "F.Cu") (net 26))
 (segment (start 141.422999 329.128999) (end 141.422999 327.086999) (width 0.25) (layer "F.Cu") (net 26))
 (segment (start 142.748 330.454) (end 141.422999 329.128999) (width 0.25) (layer "F.Cu") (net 26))
 (segment (start 116.65 332.794) (end 116.65 332.75) (width 0.25) (layer "F.Cu") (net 11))
 (segment (start 121.951001 338.095001) (end 116.65 332.794) (width 0.25) (layer "F.Cu") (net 11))
 (segment (start 113.792 350.52) (end 113.792 347.98) (width 0.25) (layer "F.Cu") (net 27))
 (segment (start 113.792 327.66) (end 113.792 325.12) (width 0.25) (layer "F.Cu") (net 27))
 (segment (start 132.842 354.33) (end 122.99 354.33) (width 0.25) (layer "F.Cu") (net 27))
 (segment (start 113.792 314.96) (end 113.792 312.42) (width 0.25) (layer "F.Cu") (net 27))
 (segment (start 113.792 332.74) (end 113.792 330.2) (width 0.25) (layer "F.Cu") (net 27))
 (segment (start 134.62 356.108) (end 132.842 354.33) (width 0.25) (layer "F.Cu") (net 27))
 (segment (start 113.792 325.12) (end 113.792 322.58) (width 0.25) (layer "F.Cu") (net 27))
 (segment (start 113.792 347.98) (end 116.64 347.98) (width 0.25) (layer "F.Cu") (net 27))
 (segment (start 113.792 317.5) (end 113.792 314.96) (width 0.25) (layer "F.Cu") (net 27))
 (segment (start 138.316002 314.565998) (end 138.316002 319.19) (width 0.25) (layer "F.Cu") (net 27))
 (segment (start 142.748 356.108) (end 134.62 356.108) (width 0.25) (layer "F.Cu") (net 27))
 (segment (start 122.99 354.33) (end 116.65 347.99) (width 0.25) (layer "F.Cu") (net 27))
 (segment (start 113.792 342.9) (end 113.792 340.36) (width 0.25) (layer "F.Cu") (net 27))
 (segment (start 113.792 340.36) (end 113.792 337.82) (width 0.25) (layer "F.Cu") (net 27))
 (segment (start 138.316002 319.19) (end 137.191001 320.315001) (width 0.25) (layer "F.Cu") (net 27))
 (segment (start 113.792 347.98) (end 113.792 345.44) (width 0.25) (layer "F.Cu") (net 27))
 (segment (start 113.792 337.82) (end 113.792 335.28) (width 0.25) (layer "F.Cu") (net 27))
 (segment (start 116.64 347.98) (end 116.65 347.99) (width 0.25) (layer "F.Cu") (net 27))
 (segment (start 113.792 322.58) (end 113.792 320.04) (width 0.25) (layer "F.Cu") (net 27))
 (segment (start 142.748 310.134) (end 138.316002 314.565998) (width 0.25) (layer "F.Cu") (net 27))
 (segment (start 113.792 345.44) (end 113.792 342.9) (width 0.25) (layer "F.Cu") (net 27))
 (segment (start 113.792 335.28) (end 113.792 332.74) (width 0.25) (layer "F.Cu") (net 27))
 (segment (start 113.792 330.2) (end 113.792 327.66) (width 0.25) (layer "F.Cu") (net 27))
 (segment (start 113.792 320.04) (end 113.792 317.5) (width 0.25) (layer "F.Cu") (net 27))
 (segment (start 113.792 313.326998) (end 113.792 320.04) (width 0.25) (layer "B.Cu") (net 27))
 (segment (start 117.751002 319.19) (end 120.581 316.360002) (width 0.25) (layer "B.Cu") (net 27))
 (segment (start 136.066 319.19) (end 117.751002 319.19) (width 0.25) (layer "B.Cu") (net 27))
 (segment (start 123.076002 311.635) (end 122.546001 311.104999) (width 0.25) (layer "B.Cu") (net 27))
 (segment (start 137.191001 320.315001) (end 136.066 319.19) (width 0.25) (layer "B.Cu") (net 27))
 (segment (start 122.491002 316.360002) (end 123.076002 315.775002) (width 0.25) (layer "B.Cu") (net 27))
 (segment (start 122.546001 311.104999) (end 116.013999 311.104999) (width 0.25) (layer "B.Cu") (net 27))
 (segment (start 116.013999 311.104999) (end 113.792 313.326998) (width 0.25) (layer "B.Cu") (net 27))
 (segment (start 120.581 316.360002) (end 122.491002 316.360002) (width 0.25) (layer "B.Cu") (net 27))
 (segment (start 123.076002 315.775002) (end 123.076002 311.635) (width 0.25) (layer "B.Cu") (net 27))
 (segment (start 116.65 335.334) (end 116.65 335.29) (width 0.25) (layer "F.Cu") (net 12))
 (segment (start 121.951001 340.635001) (end 116.65 335.334) (width 0.25) (layer "F.Cu") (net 12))
 (segment (start 121.951001 343.175001) (end 116.65 337.874) (width 0.25) (layer "F.Cu") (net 13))
 (segment (start 116.65 337.874) (end 116.65 337.83) (width 0.25) (layer "F.Cu") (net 13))
 (segment (start 116.65 340.414) (end 116.65 340.37) (width 0.25) (layer "F.Cu") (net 14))
 (segment (start 121.951001 345.715001) (end 116.65 340.414) (width 0.25) (layer "F.Cu") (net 14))
 (segment (start 135.6 305.86) (end 134.84 305.1) (width 0.25) (layer "F.Cu") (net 28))
 (segment (start 135.6 307.2) (end 135.6 305.86) (width 0.25) (layer "F.Cu") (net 28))
 (segment (start 147.4 314.5) (end 146.686 315.214) (width 0.25) (layer "F.Cu") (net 28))
 (segment (start 127 305.1) (end 132.3 305.1) (width 0.25) (layer "F.Cu") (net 28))
 (segment (start 147.4 307.2) (end 135.6 307.2) (width 0.25) (layer "F.Cu") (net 28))
 (segment (start 146.686 315.214) (end 142.748 315.214) (width 0.25) (layer "F.Cu") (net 28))
 (segment (start 147.4 307.2) (end 147.4 314.5) (width 0.25) (layer "F.Cu") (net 28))
 (segment (start 142.748 315.214) (end 139.71 315.214) (width 0.25) (layer "B.Cu") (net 28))
 (segment (start 139.71 315.214) (end 137.191001 312.695001) (width 0.25) (layer "B.Cu") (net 28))
 (segment (start 121.951001 348.255001) (end 116.65 342.954) (width 0.25) (layer "F.Cu") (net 15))
 (segment (start 116.65 342.954) (end 116.65 342.91) (width 0.25) (layer "F.Cu") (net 15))
 (segment (start 118.040002 346.840002) (end 116.65 345.45) (width 0.25) (layer "B.Cu") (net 16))
 (segment (start 137.191001 348.255001) (end 135.776002 346.840002) (width 0.25) (layer "B.Cu") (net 16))
 (segment (start 135.776002 346.840002) (end 118.040002 346.840002) (width 0.25) (layer "B.Cu") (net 16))
 (segment (start 116.078 356.616) (end 131.064 356.616) (width 0.25) (layer "F.Cu") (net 32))
 (segment (start 131.064 356.616) (end 133.096 358.648) (width 0.25) (layer "F.Cu") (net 32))
 (segment (start 133.096 358.648) (end 142.748 358.648) (width 0.25) (layer "F.Cu") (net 32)))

